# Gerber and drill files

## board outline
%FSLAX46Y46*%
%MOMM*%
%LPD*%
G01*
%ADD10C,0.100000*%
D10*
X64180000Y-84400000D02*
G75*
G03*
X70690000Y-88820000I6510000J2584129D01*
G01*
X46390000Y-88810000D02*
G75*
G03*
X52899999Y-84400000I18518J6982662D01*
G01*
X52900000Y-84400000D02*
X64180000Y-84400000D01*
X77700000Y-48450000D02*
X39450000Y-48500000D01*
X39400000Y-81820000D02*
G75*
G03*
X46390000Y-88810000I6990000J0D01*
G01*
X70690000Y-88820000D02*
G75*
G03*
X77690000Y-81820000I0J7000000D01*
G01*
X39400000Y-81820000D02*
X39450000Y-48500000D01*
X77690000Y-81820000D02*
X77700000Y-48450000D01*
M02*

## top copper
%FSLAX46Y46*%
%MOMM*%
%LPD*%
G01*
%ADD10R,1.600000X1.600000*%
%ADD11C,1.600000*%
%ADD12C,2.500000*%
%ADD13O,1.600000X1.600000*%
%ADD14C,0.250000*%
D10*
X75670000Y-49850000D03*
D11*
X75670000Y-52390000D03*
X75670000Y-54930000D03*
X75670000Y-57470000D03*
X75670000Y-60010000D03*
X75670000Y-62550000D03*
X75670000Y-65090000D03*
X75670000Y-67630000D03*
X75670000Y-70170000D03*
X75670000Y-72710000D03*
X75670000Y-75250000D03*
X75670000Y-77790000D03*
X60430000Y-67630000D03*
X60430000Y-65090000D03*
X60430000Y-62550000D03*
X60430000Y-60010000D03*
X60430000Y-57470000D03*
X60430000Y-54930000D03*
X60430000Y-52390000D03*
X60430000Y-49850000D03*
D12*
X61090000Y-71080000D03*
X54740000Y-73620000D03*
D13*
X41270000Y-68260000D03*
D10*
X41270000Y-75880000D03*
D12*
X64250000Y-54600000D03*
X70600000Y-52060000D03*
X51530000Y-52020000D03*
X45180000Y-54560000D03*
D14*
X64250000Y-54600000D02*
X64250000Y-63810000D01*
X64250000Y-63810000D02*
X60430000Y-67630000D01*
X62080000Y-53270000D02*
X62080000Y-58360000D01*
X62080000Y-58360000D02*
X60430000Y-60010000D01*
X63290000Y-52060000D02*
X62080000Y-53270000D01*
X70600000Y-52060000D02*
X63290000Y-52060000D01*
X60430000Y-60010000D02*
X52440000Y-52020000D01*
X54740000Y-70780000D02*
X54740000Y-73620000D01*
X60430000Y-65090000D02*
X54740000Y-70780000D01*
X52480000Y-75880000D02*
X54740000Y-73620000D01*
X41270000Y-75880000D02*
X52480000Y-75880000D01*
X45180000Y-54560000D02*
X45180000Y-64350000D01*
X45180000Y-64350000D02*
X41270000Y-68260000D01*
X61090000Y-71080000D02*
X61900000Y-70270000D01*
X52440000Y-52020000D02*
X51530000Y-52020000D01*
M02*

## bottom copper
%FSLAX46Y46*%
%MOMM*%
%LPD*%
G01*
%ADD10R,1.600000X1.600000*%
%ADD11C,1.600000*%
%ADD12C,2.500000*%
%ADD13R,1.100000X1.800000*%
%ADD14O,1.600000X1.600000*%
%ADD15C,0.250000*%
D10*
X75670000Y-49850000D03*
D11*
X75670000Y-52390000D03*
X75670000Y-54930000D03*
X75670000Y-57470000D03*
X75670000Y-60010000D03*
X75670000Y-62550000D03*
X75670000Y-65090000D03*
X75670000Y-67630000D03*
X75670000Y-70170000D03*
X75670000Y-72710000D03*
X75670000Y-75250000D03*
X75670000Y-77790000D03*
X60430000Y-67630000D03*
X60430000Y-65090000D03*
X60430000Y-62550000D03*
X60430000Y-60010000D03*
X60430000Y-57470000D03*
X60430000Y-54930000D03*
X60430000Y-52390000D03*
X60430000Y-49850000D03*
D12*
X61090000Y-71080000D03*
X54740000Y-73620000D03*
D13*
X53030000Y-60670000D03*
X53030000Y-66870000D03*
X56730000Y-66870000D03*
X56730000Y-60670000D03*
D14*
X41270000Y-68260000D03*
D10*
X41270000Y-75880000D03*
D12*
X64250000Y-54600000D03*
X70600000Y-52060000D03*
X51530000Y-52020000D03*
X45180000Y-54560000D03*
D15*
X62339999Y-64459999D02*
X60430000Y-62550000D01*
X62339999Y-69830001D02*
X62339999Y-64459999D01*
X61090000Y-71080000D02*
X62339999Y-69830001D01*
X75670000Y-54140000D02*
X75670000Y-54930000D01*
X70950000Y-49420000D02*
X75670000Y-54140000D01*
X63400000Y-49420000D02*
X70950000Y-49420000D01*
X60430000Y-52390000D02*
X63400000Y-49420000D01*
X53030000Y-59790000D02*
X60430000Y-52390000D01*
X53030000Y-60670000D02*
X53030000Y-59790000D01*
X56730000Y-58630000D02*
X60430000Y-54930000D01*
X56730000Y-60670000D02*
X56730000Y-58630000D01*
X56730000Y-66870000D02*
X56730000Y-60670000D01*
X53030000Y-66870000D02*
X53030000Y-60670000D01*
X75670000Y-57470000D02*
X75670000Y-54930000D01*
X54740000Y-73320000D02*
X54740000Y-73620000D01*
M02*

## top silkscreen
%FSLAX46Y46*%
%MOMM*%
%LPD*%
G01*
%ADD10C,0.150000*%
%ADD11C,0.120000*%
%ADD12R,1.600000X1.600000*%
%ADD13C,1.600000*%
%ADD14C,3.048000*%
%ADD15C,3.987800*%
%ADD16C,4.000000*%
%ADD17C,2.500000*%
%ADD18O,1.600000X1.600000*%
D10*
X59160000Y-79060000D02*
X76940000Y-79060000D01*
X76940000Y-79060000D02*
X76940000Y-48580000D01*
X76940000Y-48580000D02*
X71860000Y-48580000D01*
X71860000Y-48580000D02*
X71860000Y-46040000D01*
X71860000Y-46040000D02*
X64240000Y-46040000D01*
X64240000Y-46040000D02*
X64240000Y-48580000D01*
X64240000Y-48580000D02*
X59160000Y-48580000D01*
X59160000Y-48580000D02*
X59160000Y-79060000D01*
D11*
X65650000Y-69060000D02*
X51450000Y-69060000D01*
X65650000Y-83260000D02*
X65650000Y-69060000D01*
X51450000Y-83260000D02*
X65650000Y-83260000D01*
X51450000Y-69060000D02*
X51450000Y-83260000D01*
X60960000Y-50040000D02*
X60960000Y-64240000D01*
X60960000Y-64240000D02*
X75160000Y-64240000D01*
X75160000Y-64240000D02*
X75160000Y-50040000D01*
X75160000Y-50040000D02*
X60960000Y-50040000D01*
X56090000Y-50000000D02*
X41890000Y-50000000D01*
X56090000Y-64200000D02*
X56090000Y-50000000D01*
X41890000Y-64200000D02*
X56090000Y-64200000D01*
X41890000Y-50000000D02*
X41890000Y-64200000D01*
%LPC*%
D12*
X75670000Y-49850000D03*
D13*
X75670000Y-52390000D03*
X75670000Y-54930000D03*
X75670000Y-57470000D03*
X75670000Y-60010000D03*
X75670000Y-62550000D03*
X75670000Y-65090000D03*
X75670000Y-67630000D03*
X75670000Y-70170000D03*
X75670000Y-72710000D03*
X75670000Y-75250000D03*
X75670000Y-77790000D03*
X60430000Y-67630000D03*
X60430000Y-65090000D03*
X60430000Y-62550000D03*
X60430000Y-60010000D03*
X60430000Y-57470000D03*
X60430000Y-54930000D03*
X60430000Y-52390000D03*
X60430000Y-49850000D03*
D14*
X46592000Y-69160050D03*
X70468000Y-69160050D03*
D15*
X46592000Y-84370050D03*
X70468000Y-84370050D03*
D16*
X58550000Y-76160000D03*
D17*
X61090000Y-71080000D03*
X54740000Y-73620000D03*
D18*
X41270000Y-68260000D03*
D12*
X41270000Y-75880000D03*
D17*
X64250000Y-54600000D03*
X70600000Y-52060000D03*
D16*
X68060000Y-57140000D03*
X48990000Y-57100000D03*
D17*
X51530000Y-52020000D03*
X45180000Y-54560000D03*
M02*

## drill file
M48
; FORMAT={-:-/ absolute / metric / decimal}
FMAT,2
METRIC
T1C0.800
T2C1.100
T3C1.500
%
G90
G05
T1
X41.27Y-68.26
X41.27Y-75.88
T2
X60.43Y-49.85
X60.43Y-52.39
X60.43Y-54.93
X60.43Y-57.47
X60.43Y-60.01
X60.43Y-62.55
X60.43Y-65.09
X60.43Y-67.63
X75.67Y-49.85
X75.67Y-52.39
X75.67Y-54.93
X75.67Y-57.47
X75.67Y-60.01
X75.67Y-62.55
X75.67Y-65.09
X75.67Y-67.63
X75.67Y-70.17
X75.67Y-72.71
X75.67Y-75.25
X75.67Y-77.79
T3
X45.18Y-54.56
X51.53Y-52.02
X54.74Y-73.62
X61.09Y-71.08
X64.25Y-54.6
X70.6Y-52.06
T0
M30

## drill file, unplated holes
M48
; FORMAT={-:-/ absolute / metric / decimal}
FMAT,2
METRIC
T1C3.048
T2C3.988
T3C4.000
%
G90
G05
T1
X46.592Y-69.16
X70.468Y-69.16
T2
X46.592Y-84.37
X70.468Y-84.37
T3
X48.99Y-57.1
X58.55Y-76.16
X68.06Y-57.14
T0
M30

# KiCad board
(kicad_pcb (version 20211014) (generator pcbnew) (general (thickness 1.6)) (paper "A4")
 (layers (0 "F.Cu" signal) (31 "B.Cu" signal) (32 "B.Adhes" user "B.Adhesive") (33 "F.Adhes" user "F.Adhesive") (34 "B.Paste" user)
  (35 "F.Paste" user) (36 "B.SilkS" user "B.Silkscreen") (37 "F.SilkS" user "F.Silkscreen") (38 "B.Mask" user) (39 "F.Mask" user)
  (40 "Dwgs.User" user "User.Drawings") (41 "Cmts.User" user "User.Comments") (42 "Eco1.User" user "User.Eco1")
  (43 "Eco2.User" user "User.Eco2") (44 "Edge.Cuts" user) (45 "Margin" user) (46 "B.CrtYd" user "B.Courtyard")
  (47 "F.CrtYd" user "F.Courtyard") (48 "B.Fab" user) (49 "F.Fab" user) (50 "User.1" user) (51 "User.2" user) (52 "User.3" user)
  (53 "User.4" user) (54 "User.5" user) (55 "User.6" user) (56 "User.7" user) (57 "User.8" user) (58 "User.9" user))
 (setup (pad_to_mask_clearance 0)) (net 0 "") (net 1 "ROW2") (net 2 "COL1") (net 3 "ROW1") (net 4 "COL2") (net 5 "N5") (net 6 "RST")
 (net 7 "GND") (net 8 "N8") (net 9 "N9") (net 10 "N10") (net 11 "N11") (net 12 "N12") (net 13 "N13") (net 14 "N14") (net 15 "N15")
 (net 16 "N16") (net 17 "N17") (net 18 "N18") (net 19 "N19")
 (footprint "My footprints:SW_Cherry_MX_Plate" (layer "F.Cu") (at 68.06 57.14)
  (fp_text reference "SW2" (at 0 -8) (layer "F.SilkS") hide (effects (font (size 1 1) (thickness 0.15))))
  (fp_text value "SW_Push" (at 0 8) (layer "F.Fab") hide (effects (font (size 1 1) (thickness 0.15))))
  (fp_line (start -7.1 7.1) (end 7.1 7.1) (layer "F.SilkS") (width 0.12))
  (fp_line (start 7.1 7.1) (end 7.1 -7.1) (layer "F.SilkS") (width 0.12))
  (fp_line (start -7.1 -7.1) (end -7.1 7.1) (layer "F.SilkS") (width 0.12))
  (fp_line (start 7.1 -7.1) (end -7.1 -7.1) (layer "F.SilkS") (width 0.12))
  (pad "" np_thru_hole circle locked (at 0 0) (size 4 4) (drill 4) (layers *.Cu *.Mask))
  (pad "1" thru_hole circle locked (at -3.81 -2.54) (size 2.5 2.5) (drill 1.5) (layers *.Cu *.Mask) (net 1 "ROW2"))
  (pad "2" thru_hole circle locked (at 2.54 -5.08) (size 2.5 2.5) (drill 1.5) (layers *.Cu *.Mask) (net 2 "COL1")))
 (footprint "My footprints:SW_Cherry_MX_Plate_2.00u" (layer "F.Cu") (at 58.55 76.16)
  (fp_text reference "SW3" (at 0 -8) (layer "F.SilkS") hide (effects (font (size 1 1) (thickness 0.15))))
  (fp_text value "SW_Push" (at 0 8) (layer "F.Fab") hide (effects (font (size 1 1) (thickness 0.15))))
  (fp_line (start 7.1 7.1) (end 7.1 -7.1) (layer "F.SilkS") (width 0.12))
  (fp_line (start 7.1 -7.1) (end -7.1 -7.1) (layer "F.SilkS") (width 0.12))
  (fp_line (start -7.1 7.1) (end 7.1 7.1) (layer "F.SilkS") (width 0.12))
  (fp_line (start -7.1 -7.1) (end -7.1 7.1) (layer "F.SilkS") (width 0.12))
  (pad "" np_thru_hole circle locked (at 0 0) (size 4 4) (drill 4) (layers *.Cu *.Mask))
  (pad "1" thru_hole circle locked (at -3.81 -2.54) (size 2.5 2.5) (drill 1.5) (layers *.Cu *.Mask) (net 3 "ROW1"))
  (pad "2" thru_hole circle locked (at 2.54 -5.08) (size 2.5 2.5) (drill 1.5) (layers *.Cu *.Mask) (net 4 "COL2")))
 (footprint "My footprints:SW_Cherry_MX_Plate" (layer "F.Cu") (at 48.99 57.1)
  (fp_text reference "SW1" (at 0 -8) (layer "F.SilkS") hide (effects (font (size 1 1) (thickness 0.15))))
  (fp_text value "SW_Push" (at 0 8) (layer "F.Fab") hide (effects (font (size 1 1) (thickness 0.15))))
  (fp_line (start 7.1 7.1) (end 7.1 -7.1) (layer "F.SilkS") (width 0.12))
  (fp_line (start -7.1 7.1) (end 7.1 7.1) (layer "F.SilkS") (width 0.12))
  (fp_line (start 7.1 -7.1) (end -7.1 -7.1) (layer "F.SilkS") (width 0.12))
  (fp_line (start -7.1 -7.1) (end -7.1 7.1) (layer "F.SilkS") (width 0.12))
  (pad "" np_thru_hole circle locked (at 0 0) (size 4 4) (drill 4) (layers *.Cu *.Mask))
  (pad "1" thru_hole circle locked (at -3.81 -2.54) (size 2.5 2.5) (drill 1.5) (layers *.Cu *.Mask) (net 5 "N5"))
  (pad "2" thru_hole circle locked (at 2.54 -5.08) (size 2.5 2.5) (drill 1.5) (layers *.Cu *.Mask) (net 2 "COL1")))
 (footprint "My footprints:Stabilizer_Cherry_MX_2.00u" (layer "F.Cu") (at 58.53 76.14505)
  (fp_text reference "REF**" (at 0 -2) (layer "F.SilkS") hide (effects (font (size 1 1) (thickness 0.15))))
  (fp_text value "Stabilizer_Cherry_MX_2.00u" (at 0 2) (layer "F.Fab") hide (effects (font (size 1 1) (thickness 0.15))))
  (pad "" np_thru_hole circle locked (at 11.938 -6.985) (size 3.048 3.048) (drill 3.048) (layers *.Cu *.Mask))
  (pad "" np_thru_hole circle locked (at -11.938 -6.985) (size 3.048 3.048) (drill 3.048) (layers *.Cu *.Mask))
  (pad "" np_thru_hole circle locked (at 11.938 8.225) (size 3.9878 3.9878) (drill 3.9878) (layers *.Cu *.Mask))
  (pad "" np_thru_hole circle locked (at -11.938 8.225) (size 3.9878 3.9878) (drill 3.9878) (layers *.Cu *.Mask)))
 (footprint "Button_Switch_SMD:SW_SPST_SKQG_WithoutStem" (layer "B.Cu") (at 54.88 63.77 90)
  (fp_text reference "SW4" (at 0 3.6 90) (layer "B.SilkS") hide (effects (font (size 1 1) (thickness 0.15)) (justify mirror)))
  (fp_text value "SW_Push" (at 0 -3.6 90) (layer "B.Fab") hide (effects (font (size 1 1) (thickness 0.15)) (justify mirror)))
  (pad "1" smd rect (at -3.1 1.85 90) (size 1.8 1.1) (layers "B.Cu" "B.Paste" "B.Mask") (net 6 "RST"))
  (pad "1" smd rect (at 3.1 1.85 90) (size 1.8 1.1) (layers "B.Cu" "B.Paste" "B.Mask") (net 6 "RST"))
  (pad "2" smd rect (at -3.1 -1.85 90) (size 1.8 1.1) (layers "B.Cu" "B.Paste" "B.Mask") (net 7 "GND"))
  (pad "2" smd rect (at 3.1 -1.85 90) (size 1.8 1.1) (layers "B.Cu" "B.Paste" "B.Mask") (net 7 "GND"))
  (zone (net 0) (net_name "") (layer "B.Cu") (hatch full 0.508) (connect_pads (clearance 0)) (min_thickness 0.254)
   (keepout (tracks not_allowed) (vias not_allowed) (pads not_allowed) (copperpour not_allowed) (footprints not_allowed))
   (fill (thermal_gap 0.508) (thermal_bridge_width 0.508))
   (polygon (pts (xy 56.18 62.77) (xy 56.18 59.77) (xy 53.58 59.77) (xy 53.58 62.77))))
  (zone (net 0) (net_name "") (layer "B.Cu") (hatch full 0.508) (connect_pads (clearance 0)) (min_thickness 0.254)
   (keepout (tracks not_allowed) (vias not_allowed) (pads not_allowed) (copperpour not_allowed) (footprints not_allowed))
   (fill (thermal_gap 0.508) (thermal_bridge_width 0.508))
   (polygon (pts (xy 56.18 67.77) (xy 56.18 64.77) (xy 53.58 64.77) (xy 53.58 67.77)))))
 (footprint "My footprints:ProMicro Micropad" (layer "B.Cu") (at 68.05 63.82 -90)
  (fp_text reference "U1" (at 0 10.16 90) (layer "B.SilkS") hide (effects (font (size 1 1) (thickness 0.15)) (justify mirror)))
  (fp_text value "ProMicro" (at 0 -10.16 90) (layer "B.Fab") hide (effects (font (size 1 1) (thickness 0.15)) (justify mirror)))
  (fp_line (start -15.24 -3.81) (end -17.78 -3.81) (layer "F.SilkS") (width 0.15))
  (fp_line (start -15.24 3.81) (end -15.24 8.89) (layer "F.SilkS") (width 0.15))
  (fp_line (start -17.78 -3.81) (end -17.78 3.81) (layer "F.SilkS") (width 0.15))
  (fp_line (start -15.24 8.89) (end 15.24 8.89) (layer "F.SilkS") (width 0.15))
  (fp_line (start -15.24 -8.89) (end -15.24 -3.81) (layer "F.SilkS") (width 0.15))
  (fp_line (start 15.24 -8.89) (end -15.24 -8.89) (layer "F.SilkS") (width 0.15))
  (fp_line (start -17.78 3.81) (end -15.24 3.81) (layer "F.SilkS") (width 0.15))
  (fp_line (start 15.24 8.89) (end 15.24 -8.89) (layer "F.SilkS") (width 0.15))
  (pad "1" thru_hole rect locked (at -13.97 -7.62 270) (size 1.6 1.6) (drill 1.1) (layers *.Cu *.Mask "B.SilkS") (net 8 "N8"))
  (pad "2" thru_hole circle locked (at -11.43 -7.62 270) (size 1.6 1.6) (drill 1.1) (layers *.Cu *.Mask "B.SilkS") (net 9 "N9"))
  (pad "3" thru_hole circle locked (at -8.89 -7.62 270) (size 1.6 1.6) (drill 1.1) (layers *.Cu *.Mask "B.SilkS") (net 7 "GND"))
  (pad "4" thru_hole circle locked (at -6.35 -7.62 270) (size 1.6 1.6) (drill 1.1) (layers *.Cu *.Mask "B.SilkS") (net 7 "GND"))
  (pad "5" thru_hole circle locked (at -3.81 -7.62 270) (size 1.6 1.6) (drill 1.1) (layers *.Cu *.Mask "B.SilkS") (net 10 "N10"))
  (pad "6" thru_hole circle locked (at -1.27 -7.62 270) (size 1.6 1.6) (drill 1.1) (layers *.Cu *.Mask "B.SilkS") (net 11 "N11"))
  (pad "7" thru_hole circle locked (at 1.27 -7.62 270) (size 1.6 1.6) (drill 1.1) (layers *.Cu *.Mask "B.SilkS") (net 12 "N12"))
  (pad "8" thru_hole circle locked (at 3.81 -7.62 270) (size 1.6 1.6) (drill 1.1) (layers *.Cu *.Mask "B.SilkS") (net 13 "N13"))
  (pad "9" thru_hole circle locked (at 6.35 -7.62 270) (size 1.6 1.6) (drill 1.1) (layers *.Cu *.Mask "B.SilkS") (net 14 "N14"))
  (pad "10" thru_hole circle locked (at 8.89 -7.62 270) (size 1.6 1.6) (drill 1.1) (layers *.Cu *.Mask "B.SilkS") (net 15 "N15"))
  (pad "11" thru_hole circle locked (at 11.43 -7.62 270) (size 1.6 1.6) (drill 1.1) (layers *.Cu *.Mask "B.SilkS") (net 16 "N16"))
  (pad "12" thru_hole circle locked (at 13.97 -7.62 270) (size 1.6 1.6) (drill 1.1) (layers *.Cu *.Mask "B.SilkS") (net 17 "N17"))
  (pad "17" thru_hole circle locked (at 3.81 7.62 270) (size 1.6 1.6) (drill 1.1) (layers *.Cu *.Mask "B.SilkS") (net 1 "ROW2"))
  (pad "18" thru_hole circle locked (at 1.27 7.62 270) (size 1.6 1.6) (drill 1.1) (layers *.Cu *.Mask "B.SilkS") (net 3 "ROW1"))
  (pad "19" thru_hole circle locked (at -1.27 7.62 270) (size 1.6 1.6) (drill 1.1) (layers *.Cu *.Mask "B.SilkS") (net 4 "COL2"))
  (pad "20" thru_hole circle locked (at -3.81 7.62 270) (size 1.6 1.6) (drill 1.1) (layers *.Cu *.Mask "B.SilkS") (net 2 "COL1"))
  (pad "21" thru_hole circle locked (at -6.35 7.62 270) (size 1.6 1.6) (drill 1.1) (layers *.Cu *.Mask "B.SilkS") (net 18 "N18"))
  (pad "22" thru_hole circle locked (at -8.89 7.62 270) (size 1.6 1.6) (drill 1.1) (layers *.Cu *.Mask "B.SilkS") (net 6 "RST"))
  (pad "23" thru_hole circle locked (at -11.43 7.62 270) (size 1.6 1.6) (drill 1.1) (layers *.Cu *.Mask "B.SilkS") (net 7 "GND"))
  (pad "24" thru_hole circle locked (at -13.97 7.62 270) (size 1.6 1.6) (drill 1.1) (layers *.Cu *.Mask "B.SilkS") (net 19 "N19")))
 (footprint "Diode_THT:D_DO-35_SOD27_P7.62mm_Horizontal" (layer "B.Cu") (at 41.27 75.88 90)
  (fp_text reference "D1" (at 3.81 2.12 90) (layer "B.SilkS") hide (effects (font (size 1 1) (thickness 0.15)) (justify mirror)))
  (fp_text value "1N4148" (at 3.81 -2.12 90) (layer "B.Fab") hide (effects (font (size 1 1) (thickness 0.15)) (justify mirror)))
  (pad "1" thru_hole rect (at 0 0 90) (size 1.6 1.6) (drill 0.8) (layers *.Cu *.Mask) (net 3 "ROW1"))
  (pad "2" thru_hole oval (at 7.62 0 90) (size 1.6 1.6) (drill 0.8) (layers *.Cu *.Mask) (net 5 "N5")))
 (gr_line (start 77.7 48.45) (end 39.45 48.5) (layer "Edge.Cuts") (width 0.1))
 (gr_line (start 39.4 81.82) (end 39.45 48.5) (layer "Edge.Cuts") (width 0.1))
 (gr_arc (start 77.69 81.82) (mid 75.639747 86.769747) (end 70.69 88.82) (layer "Edge.Cuts") (width 0.1))
 (gr_line (start 52.9 84.4) (end 64.18 84.4) (layer "Edge.Cuts") (width 0.1))
 (gr_arc (start 52.899999 84.4) (mid 50.324746 87.608435) (end 46.39 88.81) (layer "Edge.Cuts") (width 0.1))
 (gr_line (start 77.69 81.82) (end 77.7 48.45) (layer "Edge.Cuts") (width 0.1))
 (gr_arc (start 46.39 88.81) (mid 41.447324 86.762676) (end 39.4 81.82) (layer "Edge.Cuts") (width 0.1))
 (gr_arc (start 70.69 88.82) (mid 66.755648 87.610584) (end 64.18 84.4) (layer "Edge.Cuts") (width 0.1))
 (segment (start 45.18 54.56) (end 45.18 64.35) (width 0.25) (layer "F.Cu") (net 5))
 (segment (start 45.18 64.35) (end 41.27 68.26) (width 0.25) (layer "F.Cu") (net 5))
 (segment (start 60.43 65.09) (end 54.74 70.78) (width 0.25) (layer "F.Cu") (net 3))
 (segment (start 54.74 70.78) (end 54.74 73.62) (width 0.25) (layer "F.Cu") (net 3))
 (segment (start 52.48 75.88) (end 54.74 73.62) (width 0.25) (layer "F.Cu") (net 3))
 (segment (start 41.27 75.88) (end 52.48 75.88) (width 0.25) (layer "F.Cu") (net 3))
 (segment (start 54.74 73.32) (end 54.74 73.62) (width 0.25) (layer "B.Cu") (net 3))
 (segment (start 60.43 60.01) (end 52.44 52.02) (width 0.25) (layer "F.Cu") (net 2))
 (segment (start 70.6 52.06) (end 63.29 52.06) (width 0.25) (layer "F.Cu") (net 2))
 (segment (start 63.29 52.06) (end 62.08 53.27) (width 0.25) (layer "F.Cu") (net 2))
 (segment (start 52.44 52.02) (end 51.53 52.02) (width 0.25) (layer "F.Cu") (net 2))
 (segment (start 62.08 58.36) (end 60.43 60.01) (width 0.25) (layer "F.Cu") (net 2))
 (segment (start 62.08 53.27) (end 62.08 58.36) (width 0.25) (layer "F.Cu") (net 2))
 (segment (start 61.09 71.08) (end 61.9 70.27) (width 0.25) (layer "F.Cu") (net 4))
 (segment (start 62.339999 64.459999) (end 60.43 62.55) (width 0.25) (layer "B.Cu") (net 4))
 (segment (start 62.339999 69.830001) (end 62.339999 64.459999) (width 0.25) (layer "B.Cu") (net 4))
 (segment (start 61.09 71.08) (end 62.339999 69.830001) (width 0.25) (layer "B.Cu") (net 4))
 (segment (start 64.25 54.6) (end 64.25 63.81) (width 0.25) (layer "F.Cu") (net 1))
 (segment (start 64.25 63.81) (end 60.43 67.63) (width 0.25) (layer "F.Cu") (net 1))
 (segment (start 56.73 66.87) (end 56.73 60.67) (width 0.25) (layer "B.Cu") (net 6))
 (segment (start 56.73 60.67) (end 56.73 58.63) (width 0.25) (layer "B.Cu") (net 6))
 (segment (start 56.73 58.63) (end 60.43 54.93) (width 0.25) (layer "B.Cu") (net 6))
 (segment (start 53.03 59.79) (end 60.43 52.39) (width 0.25) (layer "B.Cu") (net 7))
 (segment (start 53.03 66.87) (end 53.03 60.67) (width 0.25) (layer "B.Cu") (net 7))
 (segment (start 63.4 49.42) (end 70.95 49.42) (width 0.25) (layer "B.Cu") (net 7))
 (segment (start 53.03 60.67) (end 53.03 59.79) (width 0.25) (layer "B.Cu") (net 7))
 (segment (start 70.95 49.42) (end 75.67 54.14) (width 0.25) (layer "B.Cu") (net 7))
 (segment (start 75.67 54.14) (end 75.67 54.93) (width 0.25) (layer "B.Cu") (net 7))
 (segment (start 75.67 57.47) (end 75.67 54.93) (width 0.25) (layer "B.Cu") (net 7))
 (segment (start 60.43 52.39) (end 63.4 49.42) (width 0.25) (layer "B.Cu") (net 7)))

